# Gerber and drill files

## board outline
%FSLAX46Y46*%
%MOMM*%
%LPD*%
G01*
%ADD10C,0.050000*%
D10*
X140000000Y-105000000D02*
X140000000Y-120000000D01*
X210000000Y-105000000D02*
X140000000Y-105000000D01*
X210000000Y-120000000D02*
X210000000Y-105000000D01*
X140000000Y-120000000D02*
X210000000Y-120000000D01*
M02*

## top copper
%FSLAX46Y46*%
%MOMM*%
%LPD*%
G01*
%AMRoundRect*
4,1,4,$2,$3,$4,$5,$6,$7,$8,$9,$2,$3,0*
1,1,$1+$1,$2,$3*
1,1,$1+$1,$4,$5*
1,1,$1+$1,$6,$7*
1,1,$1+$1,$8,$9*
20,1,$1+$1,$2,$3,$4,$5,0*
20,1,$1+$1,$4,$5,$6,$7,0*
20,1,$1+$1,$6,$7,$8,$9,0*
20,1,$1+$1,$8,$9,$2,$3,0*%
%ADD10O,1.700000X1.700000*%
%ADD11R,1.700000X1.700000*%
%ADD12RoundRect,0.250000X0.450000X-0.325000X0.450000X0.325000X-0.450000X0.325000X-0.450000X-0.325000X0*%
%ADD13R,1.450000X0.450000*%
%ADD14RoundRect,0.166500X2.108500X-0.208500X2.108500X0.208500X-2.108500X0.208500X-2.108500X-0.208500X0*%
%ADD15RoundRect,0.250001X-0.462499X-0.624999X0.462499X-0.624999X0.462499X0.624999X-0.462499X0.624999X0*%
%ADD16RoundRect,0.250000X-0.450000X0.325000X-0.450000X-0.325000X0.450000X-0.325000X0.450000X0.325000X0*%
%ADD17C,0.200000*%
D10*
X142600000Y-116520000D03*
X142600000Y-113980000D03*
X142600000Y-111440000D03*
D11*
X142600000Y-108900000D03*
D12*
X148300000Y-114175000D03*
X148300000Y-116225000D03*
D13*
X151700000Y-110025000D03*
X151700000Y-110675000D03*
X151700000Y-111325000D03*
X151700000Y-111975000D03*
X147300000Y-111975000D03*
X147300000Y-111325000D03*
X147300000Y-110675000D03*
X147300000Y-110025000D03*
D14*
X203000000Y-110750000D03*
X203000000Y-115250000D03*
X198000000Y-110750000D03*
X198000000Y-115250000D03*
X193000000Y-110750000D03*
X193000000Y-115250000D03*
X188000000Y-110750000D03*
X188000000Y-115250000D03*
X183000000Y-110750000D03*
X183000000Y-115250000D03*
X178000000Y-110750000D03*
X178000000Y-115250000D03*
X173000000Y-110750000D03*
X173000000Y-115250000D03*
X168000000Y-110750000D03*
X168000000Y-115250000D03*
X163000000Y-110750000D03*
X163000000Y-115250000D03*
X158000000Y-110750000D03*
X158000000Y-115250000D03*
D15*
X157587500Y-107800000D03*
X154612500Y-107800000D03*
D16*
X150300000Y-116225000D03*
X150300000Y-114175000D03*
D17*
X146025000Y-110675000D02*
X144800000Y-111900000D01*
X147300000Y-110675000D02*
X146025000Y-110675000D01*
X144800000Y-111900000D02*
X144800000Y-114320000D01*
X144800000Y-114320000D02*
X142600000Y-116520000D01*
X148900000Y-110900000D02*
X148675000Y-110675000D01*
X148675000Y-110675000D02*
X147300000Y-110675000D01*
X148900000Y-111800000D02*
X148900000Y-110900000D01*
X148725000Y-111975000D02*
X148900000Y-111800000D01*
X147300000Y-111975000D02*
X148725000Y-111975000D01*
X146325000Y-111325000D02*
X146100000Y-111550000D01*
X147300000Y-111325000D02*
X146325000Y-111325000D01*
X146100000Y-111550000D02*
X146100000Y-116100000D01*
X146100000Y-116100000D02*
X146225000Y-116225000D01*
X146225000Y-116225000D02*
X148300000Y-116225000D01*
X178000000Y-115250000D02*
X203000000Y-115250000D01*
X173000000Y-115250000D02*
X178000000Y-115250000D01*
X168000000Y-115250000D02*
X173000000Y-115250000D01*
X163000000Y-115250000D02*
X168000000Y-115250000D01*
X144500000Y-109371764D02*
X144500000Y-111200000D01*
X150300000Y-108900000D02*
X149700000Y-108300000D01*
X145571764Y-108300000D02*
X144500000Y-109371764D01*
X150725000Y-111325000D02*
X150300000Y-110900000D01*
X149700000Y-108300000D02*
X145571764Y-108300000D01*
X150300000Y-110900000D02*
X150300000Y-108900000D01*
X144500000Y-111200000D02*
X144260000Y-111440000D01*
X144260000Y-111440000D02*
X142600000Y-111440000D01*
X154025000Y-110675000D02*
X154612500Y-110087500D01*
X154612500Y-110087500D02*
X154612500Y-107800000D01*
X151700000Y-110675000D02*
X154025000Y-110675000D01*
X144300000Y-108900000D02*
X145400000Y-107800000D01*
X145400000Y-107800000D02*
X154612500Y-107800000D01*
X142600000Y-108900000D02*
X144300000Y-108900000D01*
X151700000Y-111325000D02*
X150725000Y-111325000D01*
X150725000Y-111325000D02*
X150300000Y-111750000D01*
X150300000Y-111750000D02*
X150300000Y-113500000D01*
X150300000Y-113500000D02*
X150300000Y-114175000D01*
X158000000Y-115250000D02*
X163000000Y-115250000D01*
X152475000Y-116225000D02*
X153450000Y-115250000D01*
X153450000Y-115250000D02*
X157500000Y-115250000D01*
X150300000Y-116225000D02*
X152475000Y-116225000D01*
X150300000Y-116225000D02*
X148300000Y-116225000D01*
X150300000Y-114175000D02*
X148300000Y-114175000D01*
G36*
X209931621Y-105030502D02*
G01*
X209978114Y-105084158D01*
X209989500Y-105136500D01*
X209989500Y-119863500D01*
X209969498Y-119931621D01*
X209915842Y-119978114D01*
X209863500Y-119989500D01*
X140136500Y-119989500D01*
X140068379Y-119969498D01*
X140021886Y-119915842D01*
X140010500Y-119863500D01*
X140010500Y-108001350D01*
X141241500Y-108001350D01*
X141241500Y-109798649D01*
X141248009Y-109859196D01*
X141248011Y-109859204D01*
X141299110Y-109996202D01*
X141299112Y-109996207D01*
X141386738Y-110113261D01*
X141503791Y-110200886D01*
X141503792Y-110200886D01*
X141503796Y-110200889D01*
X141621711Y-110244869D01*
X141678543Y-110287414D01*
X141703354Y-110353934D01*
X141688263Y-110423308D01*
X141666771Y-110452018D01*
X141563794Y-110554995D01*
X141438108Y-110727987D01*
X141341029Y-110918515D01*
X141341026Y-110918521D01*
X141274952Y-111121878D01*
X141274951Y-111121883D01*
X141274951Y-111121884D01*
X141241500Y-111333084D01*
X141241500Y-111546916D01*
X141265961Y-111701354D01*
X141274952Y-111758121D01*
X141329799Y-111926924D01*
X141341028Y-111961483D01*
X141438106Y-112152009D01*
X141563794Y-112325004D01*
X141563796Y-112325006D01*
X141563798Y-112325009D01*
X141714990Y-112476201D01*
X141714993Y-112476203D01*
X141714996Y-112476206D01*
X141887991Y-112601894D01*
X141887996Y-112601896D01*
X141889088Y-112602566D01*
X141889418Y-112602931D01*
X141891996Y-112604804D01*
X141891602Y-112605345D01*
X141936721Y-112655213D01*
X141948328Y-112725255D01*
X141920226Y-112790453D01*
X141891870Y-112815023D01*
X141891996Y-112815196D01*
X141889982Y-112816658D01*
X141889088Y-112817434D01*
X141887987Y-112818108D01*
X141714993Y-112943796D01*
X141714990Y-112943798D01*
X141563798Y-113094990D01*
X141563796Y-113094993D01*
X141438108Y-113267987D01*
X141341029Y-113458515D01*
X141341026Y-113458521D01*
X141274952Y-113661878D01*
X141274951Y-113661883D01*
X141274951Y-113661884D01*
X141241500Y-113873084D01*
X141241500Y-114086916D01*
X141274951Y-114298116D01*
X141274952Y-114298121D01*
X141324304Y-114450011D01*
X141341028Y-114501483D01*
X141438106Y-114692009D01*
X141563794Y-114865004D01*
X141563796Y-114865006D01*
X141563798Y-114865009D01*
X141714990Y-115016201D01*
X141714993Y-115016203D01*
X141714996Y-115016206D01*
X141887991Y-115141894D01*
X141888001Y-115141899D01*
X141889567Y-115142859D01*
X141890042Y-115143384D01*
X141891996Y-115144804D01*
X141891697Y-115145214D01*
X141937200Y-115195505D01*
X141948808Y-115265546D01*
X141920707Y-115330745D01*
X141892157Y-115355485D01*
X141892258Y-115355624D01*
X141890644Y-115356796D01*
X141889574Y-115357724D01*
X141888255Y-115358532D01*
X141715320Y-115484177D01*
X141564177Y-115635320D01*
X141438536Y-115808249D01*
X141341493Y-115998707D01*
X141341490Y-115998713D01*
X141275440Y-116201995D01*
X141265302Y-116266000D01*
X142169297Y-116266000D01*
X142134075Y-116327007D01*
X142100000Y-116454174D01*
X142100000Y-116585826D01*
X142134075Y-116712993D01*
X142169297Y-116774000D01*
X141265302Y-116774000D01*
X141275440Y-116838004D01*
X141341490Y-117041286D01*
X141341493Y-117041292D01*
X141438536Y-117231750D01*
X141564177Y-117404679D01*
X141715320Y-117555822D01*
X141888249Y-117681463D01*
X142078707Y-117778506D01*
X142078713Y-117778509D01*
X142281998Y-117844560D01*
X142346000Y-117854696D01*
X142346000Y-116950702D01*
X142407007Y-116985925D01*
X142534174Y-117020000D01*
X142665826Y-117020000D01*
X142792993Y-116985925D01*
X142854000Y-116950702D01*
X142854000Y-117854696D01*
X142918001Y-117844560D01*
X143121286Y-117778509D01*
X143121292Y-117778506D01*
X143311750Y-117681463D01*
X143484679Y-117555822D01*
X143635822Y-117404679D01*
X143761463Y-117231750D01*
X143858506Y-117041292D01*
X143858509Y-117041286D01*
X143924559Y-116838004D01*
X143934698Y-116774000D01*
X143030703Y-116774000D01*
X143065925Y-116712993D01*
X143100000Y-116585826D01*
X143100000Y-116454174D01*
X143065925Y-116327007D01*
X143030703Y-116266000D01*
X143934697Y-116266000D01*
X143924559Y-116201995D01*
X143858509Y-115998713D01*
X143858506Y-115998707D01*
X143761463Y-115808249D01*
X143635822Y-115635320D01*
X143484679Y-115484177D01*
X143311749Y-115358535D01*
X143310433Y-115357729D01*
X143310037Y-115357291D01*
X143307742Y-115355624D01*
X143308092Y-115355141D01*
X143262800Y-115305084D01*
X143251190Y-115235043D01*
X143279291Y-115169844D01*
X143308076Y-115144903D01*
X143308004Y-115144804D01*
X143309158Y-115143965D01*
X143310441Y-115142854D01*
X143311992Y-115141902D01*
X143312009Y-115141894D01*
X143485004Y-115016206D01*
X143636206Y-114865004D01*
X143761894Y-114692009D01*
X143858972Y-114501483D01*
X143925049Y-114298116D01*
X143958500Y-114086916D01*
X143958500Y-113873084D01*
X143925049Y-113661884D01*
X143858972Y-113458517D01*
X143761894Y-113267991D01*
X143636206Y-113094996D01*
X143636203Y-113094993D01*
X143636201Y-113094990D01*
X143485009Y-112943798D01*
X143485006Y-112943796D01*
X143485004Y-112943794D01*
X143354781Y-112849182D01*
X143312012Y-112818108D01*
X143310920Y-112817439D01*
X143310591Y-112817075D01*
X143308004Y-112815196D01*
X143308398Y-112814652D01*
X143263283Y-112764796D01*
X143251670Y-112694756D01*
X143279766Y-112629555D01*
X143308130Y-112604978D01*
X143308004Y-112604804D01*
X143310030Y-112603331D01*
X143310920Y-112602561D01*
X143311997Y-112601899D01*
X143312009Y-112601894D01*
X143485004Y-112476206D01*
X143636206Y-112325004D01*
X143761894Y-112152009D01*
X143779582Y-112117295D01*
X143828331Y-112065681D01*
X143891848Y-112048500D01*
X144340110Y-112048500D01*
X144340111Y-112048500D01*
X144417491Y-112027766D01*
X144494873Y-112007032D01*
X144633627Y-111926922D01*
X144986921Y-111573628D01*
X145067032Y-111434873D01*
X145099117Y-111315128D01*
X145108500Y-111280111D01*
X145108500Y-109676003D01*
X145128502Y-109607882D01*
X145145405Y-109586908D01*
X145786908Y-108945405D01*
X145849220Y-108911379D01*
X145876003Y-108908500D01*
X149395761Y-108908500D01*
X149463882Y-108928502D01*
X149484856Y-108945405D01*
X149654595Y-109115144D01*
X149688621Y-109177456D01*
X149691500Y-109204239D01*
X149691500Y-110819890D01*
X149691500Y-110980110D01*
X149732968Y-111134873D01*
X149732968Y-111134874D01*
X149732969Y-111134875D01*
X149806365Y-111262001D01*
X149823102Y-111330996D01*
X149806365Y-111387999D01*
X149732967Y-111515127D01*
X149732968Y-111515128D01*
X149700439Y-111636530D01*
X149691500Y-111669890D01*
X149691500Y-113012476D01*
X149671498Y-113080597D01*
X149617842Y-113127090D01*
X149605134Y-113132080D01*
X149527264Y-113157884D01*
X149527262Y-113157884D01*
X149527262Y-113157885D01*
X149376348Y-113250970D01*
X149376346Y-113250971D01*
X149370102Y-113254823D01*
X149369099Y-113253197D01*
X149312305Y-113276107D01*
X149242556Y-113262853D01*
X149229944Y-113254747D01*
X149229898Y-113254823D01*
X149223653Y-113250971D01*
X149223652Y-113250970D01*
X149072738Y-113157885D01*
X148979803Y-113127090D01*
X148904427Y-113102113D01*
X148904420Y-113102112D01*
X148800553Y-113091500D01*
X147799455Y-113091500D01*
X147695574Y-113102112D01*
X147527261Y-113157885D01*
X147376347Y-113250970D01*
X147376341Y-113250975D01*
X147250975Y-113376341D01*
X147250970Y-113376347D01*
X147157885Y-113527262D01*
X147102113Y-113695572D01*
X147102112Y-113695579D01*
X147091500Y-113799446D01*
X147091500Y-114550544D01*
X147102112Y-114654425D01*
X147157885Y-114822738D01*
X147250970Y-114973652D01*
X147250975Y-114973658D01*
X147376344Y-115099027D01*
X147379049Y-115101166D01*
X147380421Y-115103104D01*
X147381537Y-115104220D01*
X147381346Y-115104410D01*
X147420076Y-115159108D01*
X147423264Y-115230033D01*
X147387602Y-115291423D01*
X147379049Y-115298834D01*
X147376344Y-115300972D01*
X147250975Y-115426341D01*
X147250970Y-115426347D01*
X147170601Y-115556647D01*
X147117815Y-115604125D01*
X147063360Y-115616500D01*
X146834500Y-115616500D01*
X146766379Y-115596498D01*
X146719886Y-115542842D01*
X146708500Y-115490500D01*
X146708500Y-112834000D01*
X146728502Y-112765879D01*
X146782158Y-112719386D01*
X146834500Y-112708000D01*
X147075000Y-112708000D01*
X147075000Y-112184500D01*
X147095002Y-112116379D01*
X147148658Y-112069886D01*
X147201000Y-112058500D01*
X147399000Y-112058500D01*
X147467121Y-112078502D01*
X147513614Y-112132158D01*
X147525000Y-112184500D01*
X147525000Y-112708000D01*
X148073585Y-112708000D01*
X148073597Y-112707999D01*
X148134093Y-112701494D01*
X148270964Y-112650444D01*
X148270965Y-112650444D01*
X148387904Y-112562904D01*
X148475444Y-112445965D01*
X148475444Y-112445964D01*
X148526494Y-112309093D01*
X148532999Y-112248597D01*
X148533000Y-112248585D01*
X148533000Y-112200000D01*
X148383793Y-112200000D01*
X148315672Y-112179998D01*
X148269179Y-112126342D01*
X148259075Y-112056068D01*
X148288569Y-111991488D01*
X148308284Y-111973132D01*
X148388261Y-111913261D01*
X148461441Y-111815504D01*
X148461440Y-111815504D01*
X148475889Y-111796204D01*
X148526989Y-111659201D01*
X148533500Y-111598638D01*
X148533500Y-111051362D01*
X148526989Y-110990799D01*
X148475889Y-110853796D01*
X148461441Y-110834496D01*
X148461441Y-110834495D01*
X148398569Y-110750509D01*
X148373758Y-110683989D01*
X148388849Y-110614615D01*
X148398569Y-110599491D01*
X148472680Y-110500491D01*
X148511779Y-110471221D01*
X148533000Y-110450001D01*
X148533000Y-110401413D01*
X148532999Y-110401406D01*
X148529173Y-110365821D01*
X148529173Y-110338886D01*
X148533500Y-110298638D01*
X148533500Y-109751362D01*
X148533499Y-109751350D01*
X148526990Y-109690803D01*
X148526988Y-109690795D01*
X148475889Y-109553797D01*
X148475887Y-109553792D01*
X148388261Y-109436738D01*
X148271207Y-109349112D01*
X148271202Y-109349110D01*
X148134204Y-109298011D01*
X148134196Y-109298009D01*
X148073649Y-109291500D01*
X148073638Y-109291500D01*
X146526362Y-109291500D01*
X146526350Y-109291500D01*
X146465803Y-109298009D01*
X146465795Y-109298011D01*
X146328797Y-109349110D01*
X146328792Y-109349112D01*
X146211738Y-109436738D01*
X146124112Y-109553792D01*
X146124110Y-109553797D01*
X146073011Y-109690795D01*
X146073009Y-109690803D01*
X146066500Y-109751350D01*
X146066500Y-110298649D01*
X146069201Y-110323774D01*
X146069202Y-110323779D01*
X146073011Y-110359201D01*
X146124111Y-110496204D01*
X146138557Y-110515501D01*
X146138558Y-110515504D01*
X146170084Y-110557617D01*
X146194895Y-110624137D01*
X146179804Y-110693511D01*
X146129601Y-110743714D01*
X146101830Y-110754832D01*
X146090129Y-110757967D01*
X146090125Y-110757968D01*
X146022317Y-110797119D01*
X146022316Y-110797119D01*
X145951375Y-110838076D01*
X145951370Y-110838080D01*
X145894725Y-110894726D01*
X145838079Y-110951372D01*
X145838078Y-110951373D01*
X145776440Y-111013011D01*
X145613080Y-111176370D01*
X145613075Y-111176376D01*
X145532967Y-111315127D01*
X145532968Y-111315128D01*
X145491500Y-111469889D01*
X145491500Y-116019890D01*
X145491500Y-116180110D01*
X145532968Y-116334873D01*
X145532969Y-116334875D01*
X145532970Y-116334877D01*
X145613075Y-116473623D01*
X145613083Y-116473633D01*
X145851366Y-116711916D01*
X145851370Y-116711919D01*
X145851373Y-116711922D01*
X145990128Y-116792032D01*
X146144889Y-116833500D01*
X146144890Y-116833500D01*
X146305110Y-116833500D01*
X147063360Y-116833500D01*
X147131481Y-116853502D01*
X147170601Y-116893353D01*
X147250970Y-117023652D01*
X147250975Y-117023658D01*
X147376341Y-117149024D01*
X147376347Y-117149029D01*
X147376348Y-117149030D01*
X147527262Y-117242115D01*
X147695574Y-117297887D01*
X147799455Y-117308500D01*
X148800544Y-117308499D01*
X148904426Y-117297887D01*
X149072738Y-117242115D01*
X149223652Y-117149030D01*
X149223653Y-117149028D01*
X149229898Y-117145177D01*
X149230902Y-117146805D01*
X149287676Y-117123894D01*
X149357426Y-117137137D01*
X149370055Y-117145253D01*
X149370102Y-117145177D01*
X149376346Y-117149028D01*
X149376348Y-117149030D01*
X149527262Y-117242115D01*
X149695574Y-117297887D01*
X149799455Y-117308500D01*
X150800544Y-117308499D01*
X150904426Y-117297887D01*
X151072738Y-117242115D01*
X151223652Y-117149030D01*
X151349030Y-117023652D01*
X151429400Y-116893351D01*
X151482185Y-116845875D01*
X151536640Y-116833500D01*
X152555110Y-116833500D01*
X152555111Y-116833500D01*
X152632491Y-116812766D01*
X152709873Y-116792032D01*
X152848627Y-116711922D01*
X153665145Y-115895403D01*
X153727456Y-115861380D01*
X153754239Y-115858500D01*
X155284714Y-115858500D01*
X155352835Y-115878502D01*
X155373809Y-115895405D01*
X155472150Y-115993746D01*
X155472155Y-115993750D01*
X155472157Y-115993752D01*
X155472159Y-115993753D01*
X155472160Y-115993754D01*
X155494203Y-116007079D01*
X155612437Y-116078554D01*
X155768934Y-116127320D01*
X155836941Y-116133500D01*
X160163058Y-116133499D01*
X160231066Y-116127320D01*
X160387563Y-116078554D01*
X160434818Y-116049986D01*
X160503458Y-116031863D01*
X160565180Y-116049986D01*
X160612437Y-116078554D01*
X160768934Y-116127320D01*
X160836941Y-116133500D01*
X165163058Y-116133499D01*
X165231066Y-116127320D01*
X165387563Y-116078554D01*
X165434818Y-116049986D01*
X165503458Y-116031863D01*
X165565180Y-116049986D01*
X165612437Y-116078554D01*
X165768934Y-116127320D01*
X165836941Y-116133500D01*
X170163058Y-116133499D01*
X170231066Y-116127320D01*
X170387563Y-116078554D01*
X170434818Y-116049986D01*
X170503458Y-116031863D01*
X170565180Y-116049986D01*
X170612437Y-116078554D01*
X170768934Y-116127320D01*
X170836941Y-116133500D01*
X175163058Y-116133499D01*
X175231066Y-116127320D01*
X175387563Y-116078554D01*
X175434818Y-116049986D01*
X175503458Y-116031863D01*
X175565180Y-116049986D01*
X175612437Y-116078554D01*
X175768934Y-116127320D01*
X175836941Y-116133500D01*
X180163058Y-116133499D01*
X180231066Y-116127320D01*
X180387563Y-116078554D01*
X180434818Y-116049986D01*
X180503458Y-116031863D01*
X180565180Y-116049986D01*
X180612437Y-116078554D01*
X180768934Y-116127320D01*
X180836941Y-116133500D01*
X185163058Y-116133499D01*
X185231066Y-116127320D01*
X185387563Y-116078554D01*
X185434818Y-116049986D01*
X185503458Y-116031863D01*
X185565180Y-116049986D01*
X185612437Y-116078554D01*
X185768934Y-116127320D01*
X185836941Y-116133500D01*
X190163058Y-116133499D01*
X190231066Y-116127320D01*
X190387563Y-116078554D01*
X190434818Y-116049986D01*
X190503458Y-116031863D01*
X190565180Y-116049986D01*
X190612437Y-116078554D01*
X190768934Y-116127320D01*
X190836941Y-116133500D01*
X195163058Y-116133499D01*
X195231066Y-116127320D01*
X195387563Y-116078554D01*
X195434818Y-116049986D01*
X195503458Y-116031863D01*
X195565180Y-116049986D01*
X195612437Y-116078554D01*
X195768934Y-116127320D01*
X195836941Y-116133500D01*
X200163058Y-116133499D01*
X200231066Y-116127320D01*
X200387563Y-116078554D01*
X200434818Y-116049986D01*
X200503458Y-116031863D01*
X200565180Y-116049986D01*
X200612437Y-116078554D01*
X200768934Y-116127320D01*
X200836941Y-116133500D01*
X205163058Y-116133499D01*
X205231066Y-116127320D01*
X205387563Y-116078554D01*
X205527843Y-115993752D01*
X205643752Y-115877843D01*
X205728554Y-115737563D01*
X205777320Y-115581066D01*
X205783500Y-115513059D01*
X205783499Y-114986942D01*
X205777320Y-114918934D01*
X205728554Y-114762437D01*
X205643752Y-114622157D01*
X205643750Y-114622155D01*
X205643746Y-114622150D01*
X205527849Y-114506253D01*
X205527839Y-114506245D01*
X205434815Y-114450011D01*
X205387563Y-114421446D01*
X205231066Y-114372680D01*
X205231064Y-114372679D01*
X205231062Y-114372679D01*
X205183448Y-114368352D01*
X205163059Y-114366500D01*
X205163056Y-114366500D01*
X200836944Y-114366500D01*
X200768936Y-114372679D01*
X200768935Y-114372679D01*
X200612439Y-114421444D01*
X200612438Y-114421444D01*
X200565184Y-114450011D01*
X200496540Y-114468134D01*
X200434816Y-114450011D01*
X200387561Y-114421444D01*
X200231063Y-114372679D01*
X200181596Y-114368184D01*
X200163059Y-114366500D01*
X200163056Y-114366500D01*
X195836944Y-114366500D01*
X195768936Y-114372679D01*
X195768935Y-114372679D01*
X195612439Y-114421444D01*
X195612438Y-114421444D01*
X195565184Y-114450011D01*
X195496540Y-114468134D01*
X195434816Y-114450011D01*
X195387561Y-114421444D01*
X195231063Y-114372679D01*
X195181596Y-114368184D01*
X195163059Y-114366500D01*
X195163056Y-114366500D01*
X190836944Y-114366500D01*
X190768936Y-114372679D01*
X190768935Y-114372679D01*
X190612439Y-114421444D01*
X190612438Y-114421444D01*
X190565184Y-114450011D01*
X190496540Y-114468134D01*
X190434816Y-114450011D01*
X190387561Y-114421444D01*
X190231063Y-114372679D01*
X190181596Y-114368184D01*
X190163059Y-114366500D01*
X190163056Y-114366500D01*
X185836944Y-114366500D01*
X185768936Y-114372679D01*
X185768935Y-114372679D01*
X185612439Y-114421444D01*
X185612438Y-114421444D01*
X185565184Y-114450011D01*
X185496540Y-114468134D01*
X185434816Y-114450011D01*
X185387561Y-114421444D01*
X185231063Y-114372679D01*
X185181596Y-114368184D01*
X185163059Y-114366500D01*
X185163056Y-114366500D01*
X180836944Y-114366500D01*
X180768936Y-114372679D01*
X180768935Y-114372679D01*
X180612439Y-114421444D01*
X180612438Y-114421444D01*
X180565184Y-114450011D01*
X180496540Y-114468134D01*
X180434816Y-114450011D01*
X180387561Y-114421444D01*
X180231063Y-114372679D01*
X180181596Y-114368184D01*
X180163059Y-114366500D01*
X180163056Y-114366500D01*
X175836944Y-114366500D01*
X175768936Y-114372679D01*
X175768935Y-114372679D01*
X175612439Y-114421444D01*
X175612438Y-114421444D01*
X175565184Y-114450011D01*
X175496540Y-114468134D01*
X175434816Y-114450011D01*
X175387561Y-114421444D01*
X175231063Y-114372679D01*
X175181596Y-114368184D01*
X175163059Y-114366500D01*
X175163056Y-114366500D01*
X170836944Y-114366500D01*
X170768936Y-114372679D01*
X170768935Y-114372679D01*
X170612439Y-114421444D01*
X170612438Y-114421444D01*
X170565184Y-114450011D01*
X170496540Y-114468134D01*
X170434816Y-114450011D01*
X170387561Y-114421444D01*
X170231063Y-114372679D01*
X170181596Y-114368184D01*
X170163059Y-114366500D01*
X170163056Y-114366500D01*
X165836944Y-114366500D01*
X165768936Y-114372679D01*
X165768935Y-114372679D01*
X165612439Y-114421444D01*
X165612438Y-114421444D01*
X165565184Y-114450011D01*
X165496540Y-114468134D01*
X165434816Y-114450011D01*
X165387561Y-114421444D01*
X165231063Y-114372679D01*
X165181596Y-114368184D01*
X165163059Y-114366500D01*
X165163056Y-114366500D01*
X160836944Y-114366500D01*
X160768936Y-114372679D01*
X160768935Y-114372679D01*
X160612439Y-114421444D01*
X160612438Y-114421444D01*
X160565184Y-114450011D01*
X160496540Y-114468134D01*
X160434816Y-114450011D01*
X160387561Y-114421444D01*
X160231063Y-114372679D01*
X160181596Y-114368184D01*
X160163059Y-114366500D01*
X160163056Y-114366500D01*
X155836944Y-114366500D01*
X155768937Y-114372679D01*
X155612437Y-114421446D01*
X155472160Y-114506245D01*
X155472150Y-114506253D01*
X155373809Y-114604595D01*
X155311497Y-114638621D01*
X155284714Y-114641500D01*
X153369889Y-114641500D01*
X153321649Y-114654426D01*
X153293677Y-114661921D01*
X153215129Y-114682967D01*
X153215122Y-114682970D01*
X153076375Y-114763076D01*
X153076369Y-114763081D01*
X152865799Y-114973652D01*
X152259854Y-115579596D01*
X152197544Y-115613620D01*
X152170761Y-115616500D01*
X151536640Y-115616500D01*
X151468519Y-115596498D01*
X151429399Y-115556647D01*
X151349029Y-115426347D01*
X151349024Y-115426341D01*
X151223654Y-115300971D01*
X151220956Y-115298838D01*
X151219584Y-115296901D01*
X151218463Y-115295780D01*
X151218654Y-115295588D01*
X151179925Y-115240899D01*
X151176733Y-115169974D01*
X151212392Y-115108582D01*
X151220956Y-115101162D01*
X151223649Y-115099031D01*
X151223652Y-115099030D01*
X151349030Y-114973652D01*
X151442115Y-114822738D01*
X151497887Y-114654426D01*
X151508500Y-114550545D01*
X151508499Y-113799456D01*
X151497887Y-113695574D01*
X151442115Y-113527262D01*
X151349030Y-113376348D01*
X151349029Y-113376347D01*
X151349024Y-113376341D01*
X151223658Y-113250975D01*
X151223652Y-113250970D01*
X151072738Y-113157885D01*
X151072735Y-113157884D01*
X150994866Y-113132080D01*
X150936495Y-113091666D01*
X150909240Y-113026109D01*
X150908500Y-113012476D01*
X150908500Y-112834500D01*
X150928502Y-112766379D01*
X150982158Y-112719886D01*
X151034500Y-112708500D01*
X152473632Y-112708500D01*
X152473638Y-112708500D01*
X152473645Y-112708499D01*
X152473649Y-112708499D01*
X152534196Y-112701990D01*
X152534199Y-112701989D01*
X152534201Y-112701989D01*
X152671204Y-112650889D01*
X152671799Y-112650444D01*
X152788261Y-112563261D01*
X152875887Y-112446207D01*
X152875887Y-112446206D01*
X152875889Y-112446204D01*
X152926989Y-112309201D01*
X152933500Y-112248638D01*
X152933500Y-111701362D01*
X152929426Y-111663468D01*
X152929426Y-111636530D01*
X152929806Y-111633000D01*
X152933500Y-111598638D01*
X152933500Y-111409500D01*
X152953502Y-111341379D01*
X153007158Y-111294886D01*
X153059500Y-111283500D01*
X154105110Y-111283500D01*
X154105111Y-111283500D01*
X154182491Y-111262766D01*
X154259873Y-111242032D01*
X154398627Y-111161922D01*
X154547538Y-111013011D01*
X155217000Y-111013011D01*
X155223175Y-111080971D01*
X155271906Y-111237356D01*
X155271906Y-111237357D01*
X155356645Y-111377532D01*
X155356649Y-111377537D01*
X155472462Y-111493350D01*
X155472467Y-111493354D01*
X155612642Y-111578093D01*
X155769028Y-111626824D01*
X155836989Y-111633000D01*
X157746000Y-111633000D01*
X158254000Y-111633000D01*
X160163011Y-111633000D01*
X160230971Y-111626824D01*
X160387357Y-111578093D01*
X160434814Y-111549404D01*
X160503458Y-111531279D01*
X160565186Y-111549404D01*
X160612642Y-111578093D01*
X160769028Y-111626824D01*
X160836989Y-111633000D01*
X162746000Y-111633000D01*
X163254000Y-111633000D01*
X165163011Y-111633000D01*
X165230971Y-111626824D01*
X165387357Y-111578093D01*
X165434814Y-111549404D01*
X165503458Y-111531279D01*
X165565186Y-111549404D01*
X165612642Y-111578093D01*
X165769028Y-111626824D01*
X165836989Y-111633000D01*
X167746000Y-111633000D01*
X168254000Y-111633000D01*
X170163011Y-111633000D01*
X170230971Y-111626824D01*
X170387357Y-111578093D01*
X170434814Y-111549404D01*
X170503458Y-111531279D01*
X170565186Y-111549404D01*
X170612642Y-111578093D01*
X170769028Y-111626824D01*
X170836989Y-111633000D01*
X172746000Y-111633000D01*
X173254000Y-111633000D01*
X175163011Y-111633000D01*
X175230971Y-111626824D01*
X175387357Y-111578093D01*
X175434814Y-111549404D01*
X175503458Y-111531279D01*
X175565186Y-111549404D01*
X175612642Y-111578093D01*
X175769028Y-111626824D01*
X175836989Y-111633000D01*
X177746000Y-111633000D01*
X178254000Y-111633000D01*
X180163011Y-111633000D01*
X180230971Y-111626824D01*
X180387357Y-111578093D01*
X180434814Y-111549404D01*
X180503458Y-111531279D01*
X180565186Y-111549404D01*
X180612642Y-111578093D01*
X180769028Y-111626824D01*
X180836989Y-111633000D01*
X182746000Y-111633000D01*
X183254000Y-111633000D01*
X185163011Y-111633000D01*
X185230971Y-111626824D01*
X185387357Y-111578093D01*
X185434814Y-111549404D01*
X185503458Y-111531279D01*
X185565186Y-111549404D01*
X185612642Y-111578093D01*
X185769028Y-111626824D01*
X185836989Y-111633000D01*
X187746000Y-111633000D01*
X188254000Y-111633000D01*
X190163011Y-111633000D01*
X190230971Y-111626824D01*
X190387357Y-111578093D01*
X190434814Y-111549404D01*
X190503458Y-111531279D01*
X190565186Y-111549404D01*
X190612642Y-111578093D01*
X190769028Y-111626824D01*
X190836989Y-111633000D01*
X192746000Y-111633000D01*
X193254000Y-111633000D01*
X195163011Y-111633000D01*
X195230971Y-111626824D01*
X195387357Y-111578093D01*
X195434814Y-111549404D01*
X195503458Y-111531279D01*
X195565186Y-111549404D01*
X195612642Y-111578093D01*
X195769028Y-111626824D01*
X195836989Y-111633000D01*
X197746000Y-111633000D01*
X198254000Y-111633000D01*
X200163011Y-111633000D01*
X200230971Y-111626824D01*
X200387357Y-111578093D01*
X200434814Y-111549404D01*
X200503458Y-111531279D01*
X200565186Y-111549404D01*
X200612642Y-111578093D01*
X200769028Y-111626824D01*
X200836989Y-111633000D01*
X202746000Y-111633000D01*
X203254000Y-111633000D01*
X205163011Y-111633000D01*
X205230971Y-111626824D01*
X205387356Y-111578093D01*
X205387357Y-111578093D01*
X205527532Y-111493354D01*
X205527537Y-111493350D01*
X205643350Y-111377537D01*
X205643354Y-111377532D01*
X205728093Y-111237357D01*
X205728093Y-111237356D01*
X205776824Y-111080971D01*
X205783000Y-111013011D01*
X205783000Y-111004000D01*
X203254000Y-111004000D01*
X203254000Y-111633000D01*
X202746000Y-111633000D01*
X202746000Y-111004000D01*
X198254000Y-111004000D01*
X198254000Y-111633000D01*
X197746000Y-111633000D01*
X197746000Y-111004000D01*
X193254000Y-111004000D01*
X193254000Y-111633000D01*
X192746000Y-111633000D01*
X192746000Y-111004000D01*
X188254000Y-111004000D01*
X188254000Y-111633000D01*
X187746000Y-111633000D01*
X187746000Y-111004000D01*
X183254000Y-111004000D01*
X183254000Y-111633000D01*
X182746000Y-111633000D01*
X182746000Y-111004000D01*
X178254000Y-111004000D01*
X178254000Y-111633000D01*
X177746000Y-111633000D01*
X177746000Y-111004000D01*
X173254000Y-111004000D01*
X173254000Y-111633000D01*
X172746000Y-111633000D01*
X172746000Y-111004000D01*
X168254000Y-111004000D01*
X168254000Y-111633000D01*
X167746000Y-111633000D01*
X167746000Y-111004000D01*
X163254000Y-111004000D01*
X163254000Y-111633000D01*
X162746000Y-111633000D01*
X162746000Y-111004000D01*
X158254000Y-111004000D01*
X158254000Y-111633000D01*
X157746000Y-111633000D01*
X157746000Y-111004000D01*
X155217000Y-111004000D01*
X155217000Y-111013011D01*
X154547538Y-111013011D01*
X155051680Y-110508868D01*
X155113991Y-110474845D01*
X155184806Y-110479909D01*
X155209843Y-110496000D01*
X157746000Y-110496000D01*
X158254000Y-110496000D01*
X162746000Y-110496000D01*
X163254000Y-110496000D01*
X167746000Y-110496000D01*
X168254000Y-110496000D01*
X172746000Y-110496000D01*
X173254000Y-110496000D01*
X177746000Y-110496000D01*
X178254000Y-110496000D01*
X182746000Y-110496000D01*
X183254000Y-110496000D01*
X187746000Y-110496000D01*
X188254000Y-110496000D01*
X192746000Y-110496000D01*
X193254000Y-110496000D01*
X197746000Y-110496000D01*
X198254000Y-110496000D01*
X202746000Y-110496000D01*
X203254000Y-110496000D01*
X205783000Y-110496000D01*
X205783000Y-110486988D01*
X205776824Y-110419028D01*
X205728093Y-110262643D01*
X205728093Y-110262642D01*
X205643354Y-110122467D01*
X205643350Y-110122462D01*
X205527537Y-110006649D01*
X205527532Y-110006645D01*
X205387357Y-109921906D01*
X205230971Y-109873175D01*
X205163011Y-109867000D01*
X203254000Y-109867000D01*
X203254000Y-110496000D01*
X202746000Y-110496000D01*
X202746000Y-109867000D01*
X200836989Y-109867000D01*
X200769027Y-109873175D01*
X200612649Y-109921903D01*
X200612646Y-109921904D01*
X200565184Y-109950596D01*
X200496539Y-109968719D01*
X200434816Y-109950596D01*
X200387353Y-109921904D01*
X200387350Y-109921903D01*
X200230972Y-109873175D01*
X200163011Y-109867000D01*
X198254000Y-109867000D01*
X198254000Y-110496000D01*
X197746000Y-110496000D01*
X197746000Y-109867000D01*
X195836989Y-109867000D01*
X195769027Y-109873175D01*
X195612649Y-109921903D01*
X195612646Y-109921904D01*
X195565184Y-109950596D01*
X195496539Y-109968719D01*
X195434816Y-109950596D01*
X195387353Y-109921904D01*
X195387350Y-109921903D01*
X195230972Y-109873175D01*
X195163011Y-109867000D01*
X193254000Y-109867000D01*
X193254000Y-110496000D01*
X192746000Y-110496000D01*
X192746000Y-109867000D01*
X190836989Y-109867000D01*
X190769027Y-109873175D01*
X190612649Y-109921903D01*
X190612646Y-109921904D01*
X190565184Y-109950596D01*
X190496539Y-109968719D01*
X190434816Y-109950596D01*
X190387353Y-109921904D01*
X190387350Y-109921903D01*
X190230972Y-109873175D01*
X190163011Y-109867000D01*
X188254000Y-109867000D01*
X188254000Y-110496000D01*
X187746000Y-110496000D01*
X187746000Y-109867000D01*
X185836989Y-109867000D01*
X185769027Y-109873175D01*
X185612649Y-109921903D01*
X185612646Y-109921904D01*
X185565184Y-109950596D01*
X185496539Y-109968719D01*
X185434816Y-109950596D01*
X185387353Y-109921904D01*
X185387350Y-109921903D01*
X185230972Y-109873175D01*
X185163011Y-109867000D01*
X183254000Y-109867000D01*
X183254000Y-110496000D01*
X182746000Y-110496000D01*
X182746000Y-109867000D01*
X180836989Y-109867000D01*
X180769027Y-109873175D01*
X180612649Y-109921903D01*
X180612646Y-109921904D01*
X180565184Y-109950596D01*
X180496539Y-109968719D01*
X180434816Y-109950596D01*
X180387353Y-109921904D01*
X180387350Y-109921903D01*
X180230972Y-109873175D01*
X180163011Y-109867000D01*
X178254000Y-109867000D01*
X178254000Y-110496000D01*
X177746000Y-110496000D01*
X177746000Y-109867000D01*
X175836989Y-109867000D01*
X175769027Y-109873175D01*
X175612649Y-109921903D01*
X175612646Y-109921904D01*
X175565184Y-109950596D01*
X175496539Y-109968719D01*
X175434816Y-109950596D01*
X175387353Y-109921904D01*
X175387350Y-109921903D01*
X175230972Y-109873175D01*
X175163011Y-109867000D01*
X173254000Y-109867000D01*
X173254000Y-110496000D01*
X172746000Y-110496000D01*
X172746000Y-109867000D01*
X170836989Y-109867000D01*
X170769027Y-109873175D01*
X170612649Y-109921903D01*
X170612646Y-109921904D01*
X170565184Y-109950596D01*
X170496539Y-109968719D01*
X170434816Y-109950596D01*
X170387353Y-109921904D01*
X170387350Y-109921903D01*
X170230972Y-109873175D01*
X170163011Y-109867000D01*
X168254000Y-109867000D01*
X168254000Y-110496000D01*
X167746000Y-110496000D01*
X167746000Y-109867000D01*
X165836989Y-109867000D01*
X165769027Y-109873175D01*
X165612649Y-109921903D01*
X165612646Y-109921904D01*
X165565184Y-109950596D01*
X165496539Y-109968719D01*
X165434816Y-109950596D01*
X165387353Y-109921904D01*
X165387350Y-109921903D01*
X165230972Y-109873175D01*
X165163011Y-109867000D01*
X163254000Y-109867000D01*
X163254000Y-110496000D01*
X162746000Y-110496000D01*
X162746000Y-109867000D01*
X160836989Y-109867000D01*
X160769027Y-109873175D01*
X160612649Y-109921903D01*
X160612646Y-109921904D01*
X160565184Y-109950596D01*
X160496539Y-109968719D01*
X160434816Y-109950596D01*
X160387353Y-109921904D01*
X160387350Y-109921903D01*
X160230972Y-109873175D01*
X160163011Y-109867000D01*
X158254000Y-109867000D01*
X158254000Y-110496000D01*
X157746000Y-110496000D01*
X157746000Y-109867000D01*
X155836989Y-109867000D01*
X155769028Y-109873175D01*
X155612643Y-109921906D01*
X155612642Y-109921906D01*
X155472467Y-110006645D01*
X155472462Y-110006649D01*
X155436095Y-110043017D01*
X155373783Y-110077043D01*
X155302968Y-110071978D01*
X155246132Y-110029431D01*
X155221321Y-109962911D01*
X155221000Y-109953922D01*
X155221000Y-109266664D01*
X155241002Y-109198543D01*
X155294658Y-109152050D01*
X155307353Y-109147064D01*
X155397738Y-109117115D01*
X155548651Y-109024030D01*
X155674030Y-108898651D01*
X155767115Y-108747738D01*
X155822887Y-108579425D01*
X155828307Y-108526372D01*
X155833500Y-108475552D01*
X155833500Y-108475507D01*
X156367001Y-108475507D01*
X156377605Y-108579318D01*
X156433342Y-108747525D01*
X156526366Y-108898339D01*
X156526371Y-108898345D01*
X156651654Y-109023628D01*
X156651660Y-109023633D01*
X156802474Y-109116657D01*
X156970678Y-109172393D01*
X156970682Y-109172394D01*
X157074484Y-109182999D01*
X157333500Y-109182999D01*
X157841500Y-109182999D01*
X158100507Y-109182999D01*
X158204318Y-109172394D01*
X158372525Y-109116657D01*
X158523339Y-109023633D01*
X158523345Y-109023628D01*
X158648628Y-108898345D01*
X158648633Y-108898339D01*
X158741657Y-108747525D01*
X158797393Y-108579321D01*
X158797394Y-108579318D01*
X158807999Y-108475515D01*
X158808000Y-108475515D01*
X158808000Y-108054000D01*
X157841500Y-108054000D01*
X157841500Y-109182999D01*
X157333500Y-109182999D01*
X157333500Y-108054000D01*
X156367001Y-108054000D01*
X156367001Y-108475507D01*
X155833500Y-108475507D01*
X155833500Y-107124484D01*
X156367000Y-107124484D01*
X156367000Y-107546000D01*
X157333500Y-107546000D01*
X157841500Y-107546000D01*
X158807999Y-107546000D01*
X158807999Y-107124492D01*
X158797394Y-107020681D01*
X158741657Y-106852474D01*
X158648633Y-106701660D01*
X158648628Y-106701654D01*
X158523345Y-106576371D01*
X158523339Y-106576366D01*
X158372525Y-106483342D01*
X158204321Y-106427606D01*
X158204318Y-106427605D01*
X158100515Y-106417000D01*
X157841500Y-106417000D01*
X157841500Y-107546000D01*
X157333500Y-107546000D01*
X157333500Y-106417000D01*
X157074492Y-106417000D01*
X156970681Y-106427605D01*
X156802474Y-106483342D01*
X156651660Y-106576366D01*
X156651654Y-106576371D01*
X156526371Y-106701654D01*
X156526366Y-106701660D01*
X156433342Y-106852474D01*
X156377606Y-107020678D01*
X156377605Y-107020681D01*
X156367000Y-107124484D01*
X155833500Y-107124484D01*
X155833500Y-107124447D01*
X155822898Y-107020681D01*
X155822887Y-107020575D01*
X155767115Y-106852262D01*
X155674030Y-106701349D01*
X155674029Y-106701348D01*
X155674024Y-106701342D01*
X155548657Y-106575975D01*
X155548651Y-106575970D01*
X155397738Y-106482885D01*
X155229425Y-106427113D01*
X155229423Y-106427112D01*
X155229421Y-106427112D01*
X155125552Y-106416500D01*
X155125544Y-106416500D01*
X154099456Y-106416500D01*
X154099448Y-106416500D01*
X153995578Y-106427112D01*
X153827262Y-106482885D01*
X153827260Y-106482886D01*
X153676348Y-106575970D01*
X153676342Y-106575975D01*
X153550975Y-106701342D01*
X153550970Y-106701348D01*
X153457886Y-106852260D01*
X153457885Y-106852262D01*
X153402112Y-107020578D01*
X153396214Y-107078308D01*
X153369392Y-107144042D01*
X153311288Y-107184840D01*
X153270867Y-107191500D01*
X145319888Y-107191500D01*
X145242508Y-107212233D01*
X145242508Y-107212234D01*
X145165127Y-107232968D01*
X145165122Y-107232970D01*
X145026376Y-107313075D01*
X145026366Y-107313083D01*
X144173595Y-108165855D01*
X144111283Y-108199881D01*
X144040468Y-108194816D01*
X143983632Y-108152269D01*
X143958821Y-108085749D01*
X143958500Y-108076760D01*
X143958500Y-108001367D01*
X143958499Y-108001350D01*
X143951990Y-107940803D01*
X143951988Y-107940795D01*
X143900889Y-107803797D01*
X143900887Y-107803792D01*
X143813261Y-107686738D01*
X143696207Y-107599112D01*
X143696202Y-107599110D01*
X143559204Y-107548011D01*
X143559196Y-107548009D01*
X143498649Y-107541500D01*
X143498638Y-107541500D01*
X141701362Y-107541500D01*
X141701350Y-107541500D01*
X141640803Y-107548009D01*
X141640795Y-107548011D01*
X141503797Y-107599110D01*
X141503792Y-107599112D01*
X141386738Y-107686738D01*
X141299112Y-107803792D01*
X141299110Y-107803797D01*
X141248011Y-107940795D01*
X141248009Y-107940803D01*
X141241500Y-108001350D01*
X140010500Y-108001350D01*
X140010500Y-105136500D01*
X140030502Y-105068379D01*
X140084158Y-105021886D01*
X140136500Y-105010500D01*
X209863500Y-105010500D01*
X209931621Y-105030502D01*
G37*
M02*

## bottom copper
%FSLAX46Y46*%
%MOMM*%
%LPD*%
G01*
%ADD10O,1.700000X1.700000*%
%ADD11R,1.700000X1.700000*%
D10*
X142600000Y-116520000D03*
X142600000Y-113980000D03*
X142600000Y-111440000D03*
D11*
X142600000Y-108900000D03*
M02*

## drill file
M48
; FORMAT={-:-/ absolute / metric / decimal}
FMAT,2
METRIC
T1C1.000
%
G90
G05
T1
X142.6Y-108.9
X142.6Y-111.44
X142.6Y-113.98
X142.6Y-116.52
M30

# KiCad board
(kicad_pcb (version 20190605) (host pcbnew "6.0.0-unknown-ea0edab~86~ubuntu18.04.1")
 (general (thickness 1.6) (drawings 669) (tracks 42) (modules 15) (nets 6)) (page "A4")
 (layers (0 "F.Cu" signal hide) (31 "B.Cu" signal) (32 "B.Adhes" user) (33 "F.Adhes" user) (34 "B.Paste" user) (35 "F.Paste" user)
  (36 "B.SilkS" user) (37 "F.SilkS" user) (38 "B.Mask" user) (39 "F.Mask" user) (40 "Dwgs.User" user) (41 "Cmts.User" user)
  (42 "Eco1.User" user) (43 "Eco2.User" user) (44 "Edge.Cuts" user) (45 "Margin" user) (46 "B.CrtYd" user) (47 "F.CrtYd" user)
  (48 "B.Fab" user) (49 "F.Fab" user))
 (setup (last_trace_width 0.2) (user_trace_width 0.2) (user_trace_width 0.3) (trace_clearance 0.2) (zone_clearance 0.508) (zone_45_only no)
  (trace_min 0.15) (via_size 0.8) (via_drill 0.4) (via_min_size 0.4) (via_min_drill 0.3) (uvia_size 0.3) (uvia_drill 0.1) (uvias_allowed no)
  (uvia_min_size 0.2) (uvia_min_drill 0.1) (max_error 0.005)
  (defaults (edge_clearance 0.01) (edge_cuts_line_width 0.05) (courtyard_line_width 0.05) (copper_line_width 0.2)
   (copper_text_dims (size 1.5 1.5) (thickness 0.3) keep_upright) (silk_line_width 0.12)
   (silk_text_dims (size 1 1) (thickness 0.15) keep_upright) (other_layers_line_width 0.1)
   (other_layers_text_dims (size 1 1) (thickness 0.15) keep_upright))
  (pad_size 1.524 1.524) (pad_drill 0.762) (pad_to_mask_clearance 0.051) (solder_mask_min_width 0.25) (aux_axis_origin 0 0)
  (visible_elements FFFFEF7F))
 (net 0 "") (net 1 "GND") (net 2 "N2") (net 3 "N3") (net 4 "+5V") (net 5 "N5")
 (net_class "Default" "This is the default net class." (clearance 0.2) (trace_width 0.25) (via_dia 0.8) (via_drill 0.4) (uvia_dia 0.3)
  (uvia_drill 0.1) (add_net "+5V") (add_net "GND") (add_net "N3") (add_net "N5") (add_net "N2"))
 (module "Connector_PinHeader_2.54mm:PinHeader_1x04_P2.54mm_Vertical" (layer "F.Cu") (at 142.6 108.9)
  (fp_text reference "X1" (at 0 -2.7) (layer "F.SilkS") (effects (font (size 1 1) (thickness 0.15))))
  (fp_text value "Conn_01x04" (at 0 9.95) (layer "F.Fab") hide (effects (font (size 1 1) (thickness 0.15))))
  (pad "4" thru_hole oval (at 0 7.62) (size 1.7 1.7) (drill 1) (layers *.Cu *.Mask) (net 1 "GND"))
  (pad "3" thru_hole oval (at 0 5.08) (size 1.7 1.7) (drill 1) (layers *.Cu *.Mask) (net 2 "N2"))
  (pad "2" thru_hole oval (at 0 2.54) (size 1.7 1.7) (drill 1) (layers *.Cu *.Mask) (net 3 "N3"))
  (pad "1" thru_hole rect (at 0 0) (size 1.7 1.7) (drill 1) (layers *.Cu *.Mask) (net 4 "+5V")))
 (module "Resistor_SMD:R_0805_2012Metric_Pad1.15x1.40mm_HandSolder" (layer "F.Cu") (at 148.3 115.2 90)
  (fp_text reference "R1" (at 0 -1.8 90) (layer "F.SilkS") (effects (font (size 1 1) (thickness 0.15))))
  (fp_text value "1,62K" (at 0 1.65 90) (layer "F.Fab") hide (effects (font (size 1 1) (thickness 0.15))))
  (pad "2" smd roundrect (at 1.025 0 90) (size 1.15 1.4) (layers "F.Cu" "F.Paste" "F.Mask") (roundrect_rratio 0.217391) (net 3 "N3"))
  (pad "1" smd roundrect (at -1.025 0 90) (size 1.15 1.4) (layers "F.Cu" "F.Paste" "F.Mask") (roundrect_rratio 0.217391) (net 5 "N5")))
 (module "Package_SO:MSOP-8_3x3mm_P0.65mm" (layer "F.Cu") (at 149.5 111)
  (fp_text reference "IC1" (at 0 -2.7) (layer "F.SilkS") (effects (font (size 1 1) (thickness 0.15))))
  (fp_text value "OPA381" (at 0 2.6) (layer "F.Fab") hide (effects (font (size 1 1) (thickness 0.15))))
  (pad "8" smd rect (at 2.2 -0.975) (size 1.45 0.45) (layers "F.Cu" "F.Paste" "F.Mask"))
  (pad "7" smd rect (at 2.2 -0.325) (size 1.45 0.45) (layers "F.Cu" "F.Paste" "F.Mask") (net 4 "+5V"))
  (pad "6" smd rect (at 2.2 0.325) (size 1.45 0.45) (layers "F.Cu" "F.Paste" "F.Mask") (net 3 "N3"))
  (pad "5" smd rect (at 2.2 0.975) (size 1.45 0.45) (layers "F.Cu" "F.Paste" "F.Mask"))
  (pad "4" smd rect (at -2.2 0.975) (size 1.45 0.45) (layers "F.Cu" "F.Paste" "F.Mask") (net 1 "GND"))
  (pad "3" smd rect (at -2.2 0.325) (size 1.45 0.45) (layers "F.Cu" "F.Paste" "F.Mask") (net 5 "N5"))
  (pad "2" smd rect (at -2.2 -0.325) (size 1.45 0.45) (layers "F.Cu" "F.Paste" "F.Mask") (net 1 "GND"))
  (pad "1" smd rect (at -2.2 -0.975) (size 1.45 0.45) (layers "F.Cu" "F.Paste" "F.Mask")))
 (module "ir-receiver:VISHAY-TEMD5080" (layer "F.Cu") (at 203 113 90)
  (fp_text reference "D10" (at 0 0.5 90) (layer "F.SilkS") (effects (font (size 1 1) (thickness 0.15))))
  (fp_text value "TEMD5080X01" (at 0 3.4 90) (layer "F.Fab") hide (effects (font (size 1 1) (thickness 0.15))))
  (pad "2" smd roundrect (at 2.25 0 90) (size 0.75 4.55) (layers "F.Cu" "F.Paste" "F.Mask") (roundrect_rratio 0.222) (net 1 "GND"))
  (pad "1" smd roundrect (at -2.25 0 90) (size 0.75 4.55) (layers "F.Cu" "F.Paste" "F.Mask") (roundrect_rratio 0.222) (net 5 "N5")))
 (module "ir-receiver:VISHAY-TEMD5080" (layer "F.Cu") (at 198 113 90)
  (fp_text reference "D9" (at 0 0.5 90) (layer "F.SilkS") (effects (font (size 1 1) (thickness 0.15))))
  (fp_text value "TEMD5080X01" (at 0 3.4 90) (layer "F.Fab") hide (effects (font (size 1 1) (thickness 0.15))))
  (pad "2" smd roundrect (at 2.25 0 90) (size 0.75 4.55) (layers "F.Cu" "F.Paste" "F.Mask") (roundrect_rratio 0.222) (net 1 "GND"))
  (pad "1" smd roundrect (at -2.25 0 90) (size 0.75 4.55) (layers "F.Cu" "F.Paste" "F.Mask") (roundrect_rratio 0.222) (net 5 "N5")))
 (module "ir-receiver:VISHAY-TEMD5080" (layer "F.Cu") (at 193 113 90)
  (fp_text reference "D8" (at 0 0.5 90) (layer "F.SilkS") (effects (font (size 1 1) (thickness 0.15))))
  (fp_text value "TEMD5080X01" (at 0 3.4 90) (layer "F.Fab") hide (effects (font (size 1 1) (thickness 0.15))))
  (pad "2" smd roundrect (at 2.25 0 90) (size 0.75 4.55) (layers "F.Cu" "F.Paste" "F.Mask") (roundrect_rratio 0.222) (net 1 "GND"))
  (pad "1" smd roundrect (at -2.25 0 90) (size 0.75 4.55) (layers "F.Cu" "F.Paste" "F.Mask") (roundrect_rratio 0.222) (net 5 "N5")))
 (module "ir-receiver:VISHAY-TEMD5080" (layer "F.Cu") (at 188 113 90)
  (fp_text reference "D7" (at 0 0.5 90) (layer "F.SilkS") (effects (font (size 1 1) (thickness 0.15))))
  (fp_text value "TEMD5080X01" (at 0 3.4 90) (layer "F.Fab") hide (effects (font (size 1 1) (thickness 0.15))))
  (pad "2" smd roundrect (at 2.25 0 90) (size 0.75 4.55) (layers "F.Cu" "F.Paste" "F.Mask") (roundrect_rratio 0.222) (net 1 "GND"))
  (pad "1" smd roundrect (at -2.25 0 90) (size 0.75 4.55) (layers "F.Cu" "F.Paste" "F.Mask") (roundrect_rratio 0.222) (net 5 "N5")))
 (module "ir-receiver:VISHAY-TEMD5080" (layer "F.Cu") (at 183 113 90)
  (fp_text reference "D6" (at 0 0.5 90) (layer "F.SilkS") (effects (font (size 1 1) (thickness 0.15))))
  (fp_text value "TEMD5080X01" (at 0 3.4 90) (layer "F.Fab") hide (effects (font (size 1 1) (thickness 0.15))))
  (pad "2" smd roundrect (at 2.25 0 90) (size 0.75 4.55) (layers "F.Cu" "F.Paste" "F.Mask") (roundrect_rratio 0.222) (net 1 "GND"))
  (pad "1" smd roundrect (at -2.25 0 90) (size 0.75 4.55) (layers "F.Cu" "F.Paste" "F.Mask") (roundrect_rratio 0.222) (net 5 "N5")))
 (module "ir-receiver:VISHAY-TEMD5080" (layer "F.Cu") (at 178 113 90)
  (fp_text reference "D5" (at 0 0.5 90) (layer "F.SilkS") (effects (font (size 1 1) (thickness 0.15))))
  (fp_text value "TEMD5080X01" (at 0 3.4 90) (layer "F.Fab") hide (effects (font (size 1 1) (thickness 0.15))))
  (pad "2" smd roundrect (at 2.25 0 90) (size 0.75 4.55) (layers "F.Cu" "F.Paste" "F.Mask") (roundrect_rratio 0.222) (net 1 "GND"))
  (pad "1" smd roundrect (at -2.25 0 90) (size 0.75 4.55) (layers "F.Cu" "F.Paste" "F.Mask") (roundrect_rratio 0.222) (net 5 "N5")))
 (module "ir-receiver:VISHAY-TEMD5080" (layer "F.Cu") (at 173 113 90)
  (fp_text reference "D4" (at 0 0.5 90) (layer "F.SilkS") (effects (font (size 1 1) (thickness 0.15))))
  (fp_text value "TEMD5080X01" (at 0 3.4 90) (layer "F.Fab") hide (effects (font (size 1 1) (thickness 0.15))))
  (pad "2" smd roundrect (at 2.25 0 90) (size 0.75 4.55) (layers "F.Cu" "F.Paste" "F.Mask") (roundrect_rratio 0.222) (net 1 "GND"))
  (pad "1" smd roundrect (at -2.25 0 90) (size 0.75 4.55) (layers "F.Cu" "F.Paste" "F.Mask") (roundrect_rratio 0.222) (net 5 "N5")))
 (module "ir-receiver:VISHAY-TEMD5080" (layer "F.Cu") (at 168 113 90)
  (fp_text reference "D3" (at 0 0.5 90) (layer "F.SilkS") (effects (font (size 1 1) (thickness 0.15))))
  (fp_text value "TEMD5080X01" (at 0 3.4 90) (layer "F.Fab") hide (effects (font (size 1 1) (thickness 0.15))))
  (pad "2" smd roundrect (at 2.25 0 90) (size 0.75 4.55) (layers "F.Cu" "F.Paste" "F.Mask") (roundrect_rratio 0.222) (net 1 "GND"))
  (pad "1" smd roundrect (at -2.25 0 90) (size 0.75 4.55) (layers "F.Cu" "F.Paste" "F.Mask") (roundrect_rratio 0.222) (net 5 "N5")))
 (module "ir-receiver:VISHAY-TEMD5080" (layer "F.Cu") (at 163 113 90)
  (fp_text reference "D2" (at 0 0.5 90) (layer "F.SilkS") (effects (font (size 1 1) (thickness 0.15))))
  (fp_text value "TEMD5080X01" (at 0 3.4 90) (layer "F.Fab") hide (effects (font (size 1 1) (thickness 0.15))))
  (pad "2" smd roundrect (at 2.25 0 90) (size 0.75 4.55) (layers "F.Cu" "F.Paste" "F.Mask") (roundrect_rratio 0.222) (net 1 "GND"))
  (pad "1" smd roundrect (at -2.25 0 90) (size 0.75 4.55) (layers "F.Cu" "F.Paste" "F.Mask") (roundrect_rratio 0.222) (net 5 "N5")))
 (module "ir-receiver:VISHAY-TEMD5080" (layer "F.Cu") (at 158 113 90)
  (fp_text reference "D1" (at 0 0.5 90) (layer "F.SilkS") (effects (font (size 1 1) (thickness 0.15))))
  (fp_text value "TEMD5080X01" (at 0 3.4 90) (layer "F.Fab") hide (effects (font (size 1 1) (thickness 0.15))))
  (pad "2" smd roundrect (at 2.25 0 90) (size 0.75 4.55) (layers "F.Cu" "F.Paste" "F.Mask") (roundrect_rratio 0.222) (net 1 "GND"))
  (pad "1" smd roundrect (at -2.25 0 90) (size 0.75 4.55) (layers "F.Cu" "F.Paste" "F.Mask") (roundrect_rratio 0.222) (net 5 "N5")))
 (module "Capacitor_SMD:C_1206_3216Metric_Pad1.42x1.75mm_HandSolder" (layer "F.Cu") (at 156.1 107.8)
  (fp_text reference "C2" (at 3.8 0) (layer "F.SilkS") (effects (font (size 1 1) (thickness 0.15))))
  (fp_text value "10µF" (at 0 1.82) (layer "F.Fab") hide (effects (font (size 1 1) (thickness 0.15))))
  (pad "2" smd roundrect (at 1.4875 0) (size 1.425 1.75) (layers "F.Cu" "F.Paste" "F.Mask") (roundrect_rratio 0.175439) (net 1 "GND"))
  (pad "1" smd roundrect (at -1.4875 0) (size 1.425 1.75) (layers "F.Cu" "F.Paste" "F.Mask") (roundrect_rratio 0.175439) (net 4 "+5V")))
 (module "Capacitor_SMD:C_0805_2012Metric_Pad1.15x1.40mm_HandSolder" (layer "F.Cu") (at 150.3 115.2 270)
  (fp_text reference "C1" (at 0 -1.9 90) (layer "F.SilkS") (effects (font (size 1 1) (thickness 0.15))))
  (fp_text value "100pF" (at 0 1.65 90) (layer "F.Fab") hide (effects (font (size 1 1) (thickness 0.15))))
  (pad "2" smd roundrect (at 1.025 0 270) (size 1.15 1.4) (layers "F.Cu" "F.Paste" "F.Mask") (roundrect_rratio 0.217391) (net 5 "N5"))
  (pad "1" smd roundrect (at -1.025 0 270) (size 1.15 1.4) (layers "F.Cu" "F.Paste" "F.Mask") (roundrect_rratio 0.217391) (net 3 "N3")))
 (gr_line (start 140 105) (end 140 120) (layer "Edge.Cuts") (width 0.05))
 (gr_line (start 210 105) (end 140 105) (layer "Edge.Cuts") (width 0.05))
 (gr_line (start 210 120) (end 210 105) (layer "Edge.Cuts") (width 0.05))
 (gr_line (start 140 120) (end 210 120) (layer "Edge.Cuts") (width 0.05))
 (segment (start 146.025 110.675) (end 144.8 111.9) (width 0.2) (layer "F.Cu") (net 1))
 (segment (start 147.3 110.675) (end 146.025 110.675) (width 0.2) (layer "F.Cu") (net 1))
 (segment (start 144.8 111.9) (end 144.8 114.32) (width 0.2) (layer "F.Cu") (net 1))
 (segment (start 144.8 114.32) (end 142.6 116.52) (width 0.2) (layer "F.Cu") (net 1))
 (segment (start 148.9 110.9) (end 148.675 110.675) (width 0.2) (layer "F.Cu") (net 1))
 (segment (start 148.675 110.675) (end 147.3 110.675) (width 0.2) (layer "F.Cu") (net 1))
 (segment (start 148.9 111.8) (end 148.9 110.9) (width 0.2) (layer "F.Cu") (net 1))
 (segment (start 148.725 111.975) (end 148.9 111.8) (width 0.2) (layer "F.Cu") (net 1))
 (segment (start 147.3 111.975) (end 148.725 111.975) (width 0.2) (layer "F.Cu") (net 1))
 (segment (start 146.325 111.325) (end 146.1 111.55) (width 0.2) (layer "F.Cu") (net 5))
 (segment (start 147.3 111.325) (end 146.325 111.325) (width 0.2) (layer "F.Cu") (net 5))
 (segment (start 146.1 111.55) (end 146.1 116.1) (width 0.2) (layer "F.Cu") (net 5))
 (segment (start 146.1 116.1) (end 146.225 116.225) (width 0.2) (layer "F.Cu") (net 5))
 (segment (start 146.225 116.225) (end 148.3 116.225) (width 0.2) (layer "F.Cu") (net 5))
 (segment (start 178 115.25) (end 203 115.25) (width 0.2) (layer "F.Cu") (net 5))
 (segment (start 173 115.25) (end 178 115.25) (width 0.2) (layer "F.Cu") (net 5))
 (segment (start 168 115.25) (end 173 115.25) (width 0.2) (layer "F.Cu") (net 5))
 (segment (start 163 115.25) (end 168 115.25) (width 0.2) (layer "F.Cu") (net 5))
 (segment (start 144.5 109.371764) (end 144.5 111.2) (width 0.2) (layer "F.Cu") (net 3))
 (segment (start 150.3 108.9) (end 149.7 108.3) (width 0.2) (layer "F.Cu") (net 3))
 (segment (start 145.571764 108.3) (end 144.5 109.371764) (width 0.2) (layer "F.Cu") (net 3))
 (segment (start 150.725 111.325) (end 150.3 110.9) (width 0.2) (layer "F.Cu") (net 3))
 (segment (start 149.7 108.3) (end 145.571764 108.3) (width 0.2) (layer "F.Cu") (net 3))
 (segment (start 150.3 110.9) (end 150.3 108.9) (width 0.2) (layer "F.Cu") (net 3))
 (segment (start 144.5 111.2) (end 144.26 111.44) (width 0.2) (layer "F.Cu") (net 3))
 (segment (start 144.26 111.44) (end 142.6 111.44) (width 0.2) (layer "F.Cu") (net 3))
 (segment (start 154.025 110.675) (end 154.6125 110.0875) (width 0.2) (layer "F.Cu") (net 4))
 (segment (start 154.6125 110.0875) (end 154.6125 107.8) (width 0.2) (layer "F.Cu") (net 4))
 (segment (start 151.7 110.675) (end 154.025 110.675) (width 0.2) (layer "F.Cu") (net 4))
 (segment (start 144.3 108.9) (end 145.4 107.8) (width 0.2) (layer "F.Cu") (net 4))
 (segment (start 145.4 107.8) (end 154.6125 107.8) (width 0.2) (layer "F.Cu") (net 4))
 (segment (start 142.6 108.9) (end 144.3 108.9) (width 0.2) (layer "F.Cu") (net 4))
 (segment (start 151.7 111.325) (end 150.725 111.325) (width 0.2) (layer "F.Cu") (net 3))
 (segment (start 150.725 111.325) (end 150.3 111.75) (width 0.2) (layer "F.Cu") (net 3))
 (segment (start 150.3 111.75) (end 150.3 113.5) (width 0.2) (layer "F.Cu") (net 3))
 (segment (start 150.3 113.5) (end 150.3 114.175) (width 0.2) (layer "F.Cu") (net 3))
 (segment (start 158 115.25) (end 163 115.25) (width 0.2) (layer "F.Cu") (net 5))
 (segment (start 152.475 116.225) (end 153.45 115.25) (width 0.2) (layer "F.Cu") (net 5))
 (segment (start 153.45 115.25) (end 157.5 115.25) (width 0.2) (layer "F.Cu") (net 5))
 (segment (start 150.3 116.225) (end 152.475 116.225) (width 0.2) (layer "F.Cu") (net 5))
 (segment (start 150.3 116.225) (end 148.3 116.225) (width 0.2) (layer "F.Cu") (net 5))
 (segment (start 150.3 114.175) (end 148.3 114.175) (width 0.2) (layer "F.Cu") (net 3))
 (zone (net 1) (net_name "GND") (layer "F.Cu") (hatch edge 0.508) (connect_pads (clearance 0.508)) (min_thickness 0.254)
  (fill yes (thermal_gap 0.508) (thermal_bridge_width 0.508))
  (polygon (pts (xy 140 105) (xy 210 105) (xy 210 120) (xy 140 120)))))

